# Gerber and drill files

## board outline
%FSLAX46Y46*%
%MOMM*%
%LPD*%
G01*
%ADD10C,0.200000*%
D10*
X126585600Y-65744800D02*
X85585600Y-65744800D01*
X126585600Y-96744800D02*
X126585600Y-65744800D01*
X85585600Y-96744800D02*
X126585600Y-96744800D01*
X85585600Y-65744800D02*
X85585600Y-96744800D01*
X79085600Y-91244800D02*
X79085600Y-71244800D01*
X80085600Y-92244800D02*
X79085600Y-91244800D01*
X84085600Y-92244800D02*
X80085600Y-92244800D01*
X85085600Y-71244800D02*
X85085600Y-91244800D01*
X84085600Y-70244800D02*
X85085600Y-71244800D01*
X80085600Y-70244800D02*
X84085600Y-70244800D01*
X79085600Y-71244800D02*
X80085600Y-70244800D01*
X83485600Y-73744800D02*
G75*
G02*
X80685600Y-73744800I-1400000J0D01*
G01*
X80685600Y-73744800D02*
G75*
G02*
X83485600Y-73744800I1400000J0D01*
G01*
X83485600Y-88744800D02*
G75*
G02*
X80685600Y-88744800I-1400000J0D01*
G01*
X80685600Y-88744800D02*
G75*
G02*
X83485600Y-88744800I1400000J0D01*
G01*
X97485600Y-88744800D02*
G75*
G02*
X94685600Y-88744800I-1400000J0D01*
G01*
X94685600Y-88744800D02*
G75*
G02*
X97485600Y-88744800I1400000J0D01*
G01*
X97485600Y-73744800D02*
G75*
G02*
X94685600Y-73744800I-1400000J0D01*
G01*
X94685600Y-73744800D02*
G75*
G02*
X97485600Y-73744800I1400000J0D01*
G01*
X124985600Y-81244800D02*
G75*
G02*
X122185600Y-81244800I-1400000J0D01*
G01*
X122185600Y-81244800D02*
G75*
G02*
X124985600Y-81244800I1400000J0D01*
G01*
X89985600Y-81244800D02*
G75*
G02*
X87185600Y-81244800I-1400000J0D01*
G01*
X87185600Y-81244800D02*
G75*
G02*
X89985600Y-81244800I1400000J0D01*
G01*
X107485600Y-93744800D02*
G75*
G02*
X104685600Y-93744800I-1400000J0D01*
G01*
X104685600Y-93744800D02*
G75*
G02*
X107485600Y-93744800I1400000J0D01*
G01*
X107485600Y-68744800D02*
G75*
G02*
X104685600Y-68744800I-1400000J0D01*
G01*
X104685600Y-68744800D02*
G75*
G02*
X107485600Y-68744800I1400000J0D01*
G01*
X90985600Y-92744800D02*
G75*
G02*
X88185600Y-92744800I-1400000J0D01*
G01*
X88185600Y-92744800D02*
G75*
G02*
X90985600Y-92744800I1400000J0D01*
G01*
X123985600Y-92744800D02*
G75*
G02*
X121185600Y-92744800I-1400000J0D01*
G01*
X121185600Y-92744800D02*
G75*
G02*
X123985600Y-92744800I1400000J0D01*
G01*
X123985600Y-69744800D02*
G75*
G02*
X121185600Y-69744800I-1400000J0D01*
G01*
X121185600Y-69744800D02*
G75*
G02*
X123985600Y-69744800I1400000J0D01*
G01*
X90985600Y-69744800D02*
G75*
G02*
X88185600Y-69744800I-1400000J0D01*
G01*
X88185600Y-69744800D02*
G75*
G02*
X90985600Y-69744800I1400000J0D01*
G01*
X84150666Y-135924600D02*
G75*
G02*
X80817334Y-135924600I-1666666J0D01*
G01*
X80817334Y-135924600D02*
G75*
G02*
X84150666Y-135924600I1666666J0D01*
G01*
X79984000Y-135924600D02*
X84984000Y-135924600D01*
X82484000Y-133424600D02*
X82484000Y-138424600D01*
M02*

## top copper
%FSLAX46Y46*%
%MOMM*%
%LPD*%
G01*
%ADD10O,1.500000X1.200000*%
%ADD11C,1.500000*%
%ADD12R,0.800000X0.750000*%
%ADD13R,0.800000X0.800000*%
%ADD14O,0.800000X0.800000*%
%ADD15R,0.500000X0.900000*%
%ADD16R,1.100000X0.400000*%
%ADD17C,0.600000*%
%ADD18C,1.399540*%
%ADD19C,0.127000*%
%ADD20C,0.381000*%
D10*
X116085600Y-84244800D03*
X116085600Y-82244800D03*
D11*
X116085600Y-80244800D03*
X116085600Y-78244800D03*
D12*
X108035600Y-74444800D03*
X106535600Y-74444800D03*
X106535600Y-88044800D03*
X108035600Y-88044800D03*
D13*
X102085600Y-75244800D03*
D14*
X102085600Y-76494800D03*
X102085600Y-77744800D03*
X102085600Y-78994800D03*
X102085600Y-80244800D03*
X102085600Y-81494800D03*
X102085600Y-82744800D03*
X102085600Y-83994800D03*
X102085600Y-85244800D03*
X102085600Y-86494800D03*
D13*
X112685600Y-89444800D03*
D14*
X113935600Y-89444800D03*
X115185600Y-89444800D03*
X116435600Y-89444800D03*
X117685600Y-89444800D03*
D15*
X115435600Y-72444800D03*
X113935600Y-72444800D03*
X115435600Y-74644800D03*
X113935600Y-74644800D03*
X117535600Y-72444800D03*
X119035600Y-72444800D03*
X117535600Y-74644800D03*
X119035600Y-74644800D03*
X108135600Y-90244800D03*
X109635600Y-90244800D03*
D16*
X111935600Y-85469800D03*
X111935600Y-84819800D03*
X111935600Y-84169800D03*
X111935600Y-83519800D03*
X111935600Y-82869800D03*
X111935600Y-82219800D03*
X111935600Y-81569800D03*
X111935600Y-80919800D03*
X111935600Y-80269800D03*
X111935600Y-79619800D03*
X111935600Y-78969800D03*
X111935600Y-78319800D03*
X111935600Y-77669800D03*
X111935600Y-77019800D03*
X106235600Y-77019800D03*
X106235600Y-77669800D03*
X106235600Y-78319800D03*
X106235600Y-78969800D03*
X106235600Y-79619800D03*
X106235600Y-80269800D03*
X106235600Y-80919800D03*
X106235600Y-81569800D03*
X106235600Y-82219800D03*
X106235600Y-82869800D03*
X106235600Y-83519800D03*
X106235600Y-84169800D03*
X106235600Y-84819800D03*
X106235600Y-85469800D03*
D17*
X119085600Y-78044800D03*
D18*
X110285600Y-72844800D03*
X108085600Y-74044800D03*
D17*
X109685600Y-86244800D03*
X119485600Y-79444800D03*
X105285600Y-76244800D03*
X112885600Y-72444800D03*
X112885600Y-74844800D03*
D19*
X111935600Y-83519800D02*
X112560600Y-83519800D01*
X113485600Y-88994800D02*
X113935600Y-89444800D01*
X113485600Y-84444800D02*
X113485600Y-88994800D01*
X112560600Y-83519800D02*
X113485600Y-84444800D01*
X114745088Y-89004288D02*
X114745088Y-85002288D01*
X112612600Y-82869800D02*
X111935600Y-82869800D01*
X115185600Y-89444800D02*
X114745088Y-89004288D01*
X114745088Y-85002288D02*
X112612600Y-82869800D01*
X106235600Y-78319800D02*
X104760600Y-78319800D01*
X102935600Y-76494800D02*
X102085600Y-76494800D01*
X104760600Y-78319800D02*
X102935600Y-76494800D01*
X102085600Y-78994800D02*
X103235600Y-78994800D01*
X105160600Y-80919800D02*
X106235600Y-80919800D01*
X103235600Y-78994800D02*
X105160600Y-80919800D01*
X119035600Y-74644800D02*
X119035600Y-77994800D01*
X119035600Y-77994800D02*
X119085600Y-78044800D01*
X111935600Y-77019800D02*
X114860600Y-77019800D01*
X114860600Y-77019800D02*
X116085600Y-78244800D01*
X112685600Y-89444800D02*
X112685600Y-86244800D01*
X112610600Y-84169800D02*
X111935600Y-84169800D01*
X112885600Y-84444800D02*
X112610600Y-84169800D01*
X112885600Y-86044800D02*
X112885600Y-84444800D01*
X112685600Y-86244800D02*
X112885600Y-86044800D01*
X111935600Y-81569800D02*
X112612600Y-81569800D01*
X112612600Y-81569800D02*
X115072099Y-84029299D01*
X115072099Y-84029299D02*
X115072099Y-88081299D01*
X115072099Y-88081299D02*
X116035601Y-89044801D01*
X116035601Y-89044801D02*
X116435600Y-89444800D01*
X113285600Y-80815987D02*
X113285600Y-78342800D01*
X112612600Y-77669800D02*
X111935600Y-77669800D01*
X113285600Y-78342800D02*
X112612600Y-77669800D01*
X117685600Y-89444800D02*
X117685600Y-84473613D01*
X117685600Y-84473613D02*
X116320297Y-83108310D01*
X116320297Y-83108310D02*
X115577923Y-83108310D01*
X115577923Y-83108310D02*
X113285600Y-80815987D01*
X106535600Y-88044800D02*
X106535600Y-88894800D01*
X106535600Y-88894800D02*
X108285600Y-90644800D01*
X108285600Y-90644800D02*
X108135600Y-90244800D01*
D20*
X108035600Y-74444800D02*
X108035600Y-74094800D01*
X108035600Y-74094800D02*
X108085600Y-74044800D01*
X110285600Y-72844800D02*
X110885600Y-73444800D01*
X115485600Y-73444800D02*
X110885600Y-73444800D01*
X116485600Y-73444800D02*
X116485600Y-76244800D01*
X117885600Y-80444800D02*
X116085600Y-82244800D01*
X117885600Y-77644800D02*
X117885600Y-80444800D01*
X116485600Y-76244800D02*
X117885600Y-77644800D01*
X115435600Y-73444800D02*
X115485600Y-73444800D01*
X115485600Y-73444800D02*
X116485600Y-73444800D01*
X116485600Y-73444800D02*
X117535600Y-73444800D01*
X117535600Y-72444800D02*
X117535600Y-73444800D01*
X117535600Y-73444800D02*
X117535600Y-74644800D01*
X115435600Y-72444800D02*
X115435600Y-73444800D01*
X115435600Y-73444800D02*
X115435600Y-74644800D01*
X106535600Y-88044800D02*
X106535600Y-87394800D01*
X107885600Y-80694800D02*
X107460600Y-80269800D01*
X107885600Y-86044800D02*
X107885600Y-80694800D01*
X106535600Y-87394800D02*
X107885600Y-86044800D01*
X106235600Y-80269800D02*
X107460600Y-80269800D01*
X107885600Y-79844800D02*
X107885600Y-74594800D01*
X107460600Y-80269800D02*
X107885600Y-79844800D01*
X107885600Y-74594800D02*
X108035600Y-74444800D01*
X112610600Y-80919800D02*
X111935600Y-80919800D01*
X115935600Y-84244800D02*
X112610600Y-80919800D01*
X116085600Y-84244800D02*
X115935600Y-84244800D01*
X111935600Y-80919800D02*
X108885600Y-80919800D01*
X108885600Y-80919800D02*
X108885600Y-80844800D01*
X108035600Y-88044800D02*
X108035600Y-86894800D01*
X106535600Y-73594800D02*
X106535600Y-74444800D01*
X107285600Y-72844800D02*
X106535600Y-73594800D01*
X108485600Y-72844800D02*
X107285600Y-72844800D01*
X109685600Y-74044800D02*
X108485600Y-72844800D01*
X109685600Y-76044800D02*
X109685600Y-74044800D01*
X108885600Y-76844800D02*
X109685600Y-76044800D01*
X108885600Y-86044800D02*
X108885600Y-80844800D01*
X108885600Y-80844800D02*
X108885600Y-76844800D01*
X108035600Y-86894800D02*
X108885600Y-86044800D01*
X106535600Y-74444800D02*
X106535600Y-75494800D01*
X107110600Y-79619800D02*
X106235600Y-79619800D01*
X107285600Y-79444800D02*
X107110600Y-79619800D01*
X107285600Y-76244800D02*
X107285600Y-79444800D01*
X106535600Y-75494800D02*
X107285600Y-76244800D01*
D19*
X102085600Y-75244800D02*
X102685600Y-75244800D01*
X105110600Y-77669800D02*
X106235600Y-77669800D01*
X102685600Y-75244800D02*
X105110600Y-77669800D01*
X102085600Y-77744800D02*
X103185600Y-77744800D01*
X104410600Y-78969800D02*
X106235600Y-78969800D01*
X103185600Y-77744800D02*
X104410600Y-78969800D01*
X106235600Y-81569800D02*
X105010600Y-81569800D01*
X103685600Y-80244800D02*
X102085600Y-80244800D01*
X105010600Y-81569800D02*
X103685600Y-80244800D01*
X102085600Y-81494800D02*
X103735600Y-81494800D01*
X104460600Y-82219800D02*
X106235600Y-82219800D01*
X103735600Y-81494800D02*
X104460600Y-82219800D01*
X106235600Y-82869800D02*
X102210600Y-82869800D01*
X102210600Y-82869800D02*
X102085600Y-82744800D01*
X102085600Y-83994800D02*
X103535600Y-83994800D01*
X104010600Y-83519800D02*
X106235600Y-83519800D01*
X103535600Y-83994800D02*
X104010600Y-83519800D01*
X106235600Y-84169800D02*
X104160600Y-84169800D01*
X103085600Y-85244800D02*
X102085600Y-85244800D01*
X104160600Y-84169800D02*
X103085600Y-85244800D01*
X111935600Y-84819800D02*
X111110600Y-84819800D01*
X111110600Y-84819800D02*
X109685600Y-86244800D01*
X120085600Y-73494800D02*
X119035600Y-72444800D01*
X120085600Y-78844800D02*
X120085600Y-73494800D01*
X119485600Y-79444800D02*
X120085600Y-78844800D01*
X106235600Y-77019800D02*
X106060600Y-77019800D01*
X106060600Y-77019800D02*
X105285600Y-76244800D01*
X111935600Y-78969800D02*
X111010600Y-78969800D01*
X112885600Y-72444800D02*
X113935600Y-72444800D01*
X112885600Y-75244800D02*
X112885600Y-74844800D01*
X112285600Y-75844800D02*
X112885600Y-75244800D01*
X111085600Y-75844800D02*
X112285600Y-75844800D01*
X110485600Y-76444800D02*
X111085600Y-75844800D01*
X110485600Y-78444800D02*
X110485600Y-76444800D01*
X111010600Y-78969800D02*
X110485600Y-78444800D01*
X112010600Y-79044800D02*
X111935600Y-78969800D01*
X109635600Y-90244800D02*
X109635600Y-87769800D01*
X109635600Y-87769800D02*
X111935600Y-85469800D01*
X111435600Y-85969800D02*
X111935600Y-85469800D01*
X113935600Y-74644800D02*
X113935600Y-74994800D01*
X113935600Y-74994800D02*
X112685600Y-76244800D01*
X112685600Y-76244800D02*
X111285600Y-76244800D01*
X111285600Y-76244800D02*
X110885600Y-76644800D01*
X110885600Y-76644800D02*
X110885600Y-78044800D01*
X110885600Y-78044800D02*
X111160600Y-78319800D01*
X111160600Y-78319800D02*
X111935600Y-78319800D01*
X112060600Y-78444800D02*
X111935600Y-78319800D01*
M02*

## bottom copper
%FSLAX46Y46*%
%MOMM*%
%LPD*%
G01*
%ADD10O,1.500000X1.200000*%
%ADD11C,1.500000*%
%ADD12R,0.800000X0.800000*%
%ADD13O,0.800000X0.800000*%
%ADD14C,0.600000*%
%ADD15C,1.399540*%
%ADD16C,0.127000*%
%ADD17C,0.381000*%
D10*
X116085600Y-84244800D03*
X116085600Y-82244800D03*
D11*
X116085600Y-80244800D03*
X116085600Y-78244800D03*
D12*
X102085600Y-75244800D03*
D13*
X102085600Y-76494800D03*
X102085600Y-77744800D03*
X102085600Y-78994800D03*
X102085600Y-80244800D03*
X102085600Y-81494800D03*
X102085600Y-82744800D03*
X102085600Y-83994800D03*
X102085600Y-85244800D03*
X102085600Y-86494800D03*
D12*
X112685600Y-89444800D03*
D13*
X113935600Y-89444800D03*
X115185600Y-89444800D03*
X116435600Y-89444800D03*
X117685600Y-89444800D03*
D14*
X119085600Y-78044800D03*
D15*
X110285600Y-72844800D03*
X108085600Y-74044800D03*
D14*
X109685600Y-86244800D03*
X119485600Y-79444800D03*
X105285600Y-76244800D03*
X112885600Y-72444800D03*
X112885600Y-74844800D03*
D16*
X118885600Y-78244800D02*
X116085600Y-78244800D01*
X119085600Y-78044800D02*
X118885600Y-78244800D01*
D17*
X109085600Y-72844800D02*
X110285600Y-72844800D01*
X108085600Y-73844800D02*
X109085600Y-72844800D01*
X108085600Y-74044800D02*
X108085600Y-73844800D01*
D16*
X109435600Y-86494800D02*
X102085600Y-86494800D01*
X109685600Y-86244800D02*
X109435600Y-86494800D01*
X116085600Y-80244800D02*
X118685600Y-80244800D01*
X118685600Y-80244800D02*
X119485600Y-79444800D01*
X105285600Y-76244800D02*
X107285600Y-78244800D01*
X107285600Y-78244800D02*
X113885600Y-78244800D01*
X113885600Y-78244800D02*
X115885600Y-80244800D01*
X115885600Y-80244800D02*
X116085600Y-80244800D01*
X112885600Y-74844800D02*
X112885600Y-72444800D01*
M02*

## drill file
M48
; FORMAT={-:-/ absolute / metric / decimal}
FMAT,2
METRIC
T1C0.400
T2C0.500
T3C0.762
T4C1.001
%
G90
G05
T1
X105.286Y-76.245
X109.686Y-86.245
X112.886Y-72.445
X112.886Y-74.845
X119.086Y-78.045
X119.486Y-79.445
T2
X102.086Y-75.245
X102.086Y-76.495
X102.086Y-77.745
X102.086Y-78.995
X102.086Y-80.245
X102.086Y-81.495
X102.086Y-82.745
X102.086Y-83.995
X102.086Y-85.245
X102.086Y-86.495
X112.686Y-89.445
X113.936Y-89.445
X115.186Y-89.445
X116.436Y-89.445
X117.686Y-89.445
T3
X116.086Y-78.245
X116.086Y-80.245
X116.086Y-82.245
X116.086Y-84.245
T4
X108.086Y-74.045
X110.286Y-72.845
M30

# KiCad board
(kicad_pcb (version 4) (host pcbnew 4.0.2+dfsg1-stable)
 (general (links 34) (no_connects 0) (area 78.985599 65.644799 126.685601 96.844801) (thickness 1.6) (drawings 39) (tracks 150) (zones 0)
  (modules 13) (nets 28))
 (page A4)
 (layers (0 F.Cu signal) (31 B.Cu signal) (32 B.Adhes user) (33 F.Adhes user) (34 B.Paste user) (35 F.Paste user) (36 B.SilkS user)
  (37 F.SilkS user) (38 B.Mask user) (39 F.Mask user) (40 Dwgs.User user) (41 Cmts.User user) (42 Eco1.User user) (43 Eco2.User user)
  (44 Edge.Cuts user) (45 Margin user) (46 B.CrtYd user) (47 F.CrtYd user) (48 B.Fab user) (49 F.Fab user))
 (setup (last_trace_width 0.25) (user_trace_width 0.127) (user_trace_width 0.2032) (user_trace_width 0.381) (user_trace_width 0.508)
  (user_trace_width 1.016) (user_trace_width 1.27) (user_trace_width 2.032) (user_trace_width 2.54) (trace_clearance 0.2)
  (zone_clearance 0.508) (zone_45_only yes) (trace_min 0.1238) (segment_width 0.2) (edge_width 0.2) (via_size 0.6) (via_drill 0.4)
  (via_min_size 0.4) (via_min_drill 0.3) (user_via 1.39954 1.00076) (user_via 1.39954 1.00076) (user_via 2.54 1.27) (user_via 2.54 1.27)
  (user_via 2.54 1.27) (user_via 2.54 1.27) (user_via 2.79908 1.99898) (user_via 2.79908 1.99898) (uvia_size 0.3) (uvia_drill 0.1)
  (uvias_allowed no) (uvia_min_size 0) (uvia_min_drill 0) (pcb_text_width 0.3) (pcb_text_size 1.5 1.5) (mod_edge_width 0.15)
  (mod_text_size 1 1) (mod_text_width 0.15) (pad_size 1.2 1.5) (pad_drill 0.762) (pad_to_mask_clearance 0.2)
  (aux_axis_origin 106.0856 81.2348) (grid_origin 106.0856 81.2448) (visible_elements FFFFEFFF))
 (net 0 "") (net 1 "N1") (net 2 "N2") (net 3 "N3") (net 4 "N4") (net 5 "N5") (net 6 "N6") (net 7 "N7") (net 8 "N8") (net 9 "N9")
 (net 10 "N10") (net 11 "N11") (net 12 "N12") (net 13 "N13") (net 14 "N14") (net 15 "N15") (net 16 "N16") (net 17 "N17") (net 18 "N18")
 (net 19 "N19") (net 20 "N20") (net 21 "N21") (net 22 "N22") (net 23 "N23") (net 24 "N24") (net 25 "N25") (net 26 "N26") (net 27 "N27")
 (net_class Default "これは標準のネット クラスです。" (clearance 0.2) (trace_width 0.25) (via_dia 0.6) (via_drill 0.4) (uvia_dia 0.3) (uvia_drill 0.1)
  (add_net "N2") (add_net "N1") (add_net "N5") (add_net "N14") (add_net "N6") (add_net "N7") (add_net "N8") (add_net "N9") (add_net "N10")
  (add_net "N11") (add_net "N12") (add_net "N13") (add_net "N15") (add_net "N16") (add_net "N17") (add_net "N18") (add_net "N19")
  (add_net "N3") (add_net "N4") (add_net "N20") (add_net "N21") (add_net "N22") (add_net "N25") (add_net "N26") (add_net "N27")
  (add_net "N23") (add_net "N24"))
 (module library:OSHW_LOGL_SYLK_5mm (layer F.Cu) (at 82.0856 81.2448 270)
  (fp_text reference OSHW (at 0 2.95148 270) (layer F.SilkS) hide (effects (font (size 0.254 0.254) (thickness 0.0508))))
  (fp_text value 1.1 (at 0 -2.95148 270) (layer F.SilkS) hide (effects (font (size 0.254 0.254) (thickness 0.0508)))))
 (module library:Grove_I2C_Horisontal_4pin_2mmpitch (layer F.Cu) (at 116.0856 81.2448 90)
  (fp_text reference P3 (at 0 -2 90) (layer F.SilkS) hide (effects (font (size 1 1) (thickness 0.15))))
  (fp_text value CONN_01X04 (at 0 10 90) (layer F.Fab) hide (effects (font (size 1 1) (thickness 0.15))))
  (pad 1 thru_hole oval (at -3 0 90) (size 1.2 1.5) (drill 0.762) (layers *.Cu *.Mask F.SilkS) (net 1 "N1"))
  (pad 2 thru_hole oval (at -1 0 90) (size 1.2 1.5) (drill 0.762) (layers *.Cu *.Mask F.SilkS) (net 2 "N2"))
  (pad 3 thru_hole circle (at 1 0 90) (size 1.5 1.5) (drill 0.762) (layers *.Cu *.Mask F.SilkS) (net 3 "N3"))
  (pad 4 thru_hole circle (at 3 0 90) (size 1.5 1.5) (drill 0.762) (layers *.Cu *.Mask F.SilkS) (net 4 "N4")))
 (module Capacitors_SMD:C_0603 (layer F.Cu) (at 107.2856 74.4448 180)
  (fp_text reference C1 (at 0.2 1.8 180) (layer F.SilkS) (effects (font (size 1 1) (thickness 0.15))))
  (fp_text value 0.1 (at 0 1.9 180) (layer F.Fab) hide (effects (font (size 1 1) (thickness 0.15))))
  (pad 1 smd rect (at -0.75 0 180) (size 0.8 0.75) (layers F.Cu F.Paste F.Mask) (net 2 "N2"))
  (pad 2 smd rect (at 0.75 0 180) (size 0.8 0.75) (layers F.Cu F.Paste F.Mask) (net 1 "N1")))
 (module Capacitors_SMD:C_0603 (layer F.Cu) (at 107.2856 88.0448)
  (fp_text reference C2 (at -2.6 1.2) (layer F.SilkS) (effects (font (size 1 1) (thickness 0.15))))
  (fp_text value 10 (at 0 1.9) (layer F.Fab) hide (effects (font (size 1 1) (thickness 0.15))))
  (pad 1 smd rect (at -0.75 0) (size 0.8 0.75) (layers F.Cu F.Paste F.Mask) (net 2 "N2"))
  (pad 2 smd rect (at 0.75 0) (size 0.8 0.75) (layers F.Cu F.Paste F.Mask) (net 1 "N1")))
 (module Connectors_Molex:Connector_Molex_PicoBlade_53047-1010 (layer F.Cu) (at 102.0856 75.2448 270)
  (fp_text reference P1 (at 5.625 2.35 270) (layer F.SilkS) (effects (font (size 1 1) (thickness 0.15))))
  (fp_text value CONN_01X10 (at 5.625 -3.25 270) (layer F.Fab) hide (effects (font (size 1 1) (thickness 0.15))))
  (pad 1 thru_hole rect (at 0 0 270) (size 0.8 0.8) (drill 0.5) (layers *.Cu *.Mask F.SilkS) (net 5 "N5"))
  (pad 2 thru_hole oval (at 1.25 0 270) (size 0.8 0.8) (drill 0.5) (layers *.Cu *.Mask F.SilkS) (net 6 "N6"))
  (pad 3 thru_hole oval (at 2.5 0 270) (size 0.8 0.8) (drill 0.5) (layers *.Cu *.Mask F.SilkS) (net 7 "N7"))
  (pad 4 thru_hole oval (at 3.75 0 270) (size 0.8 0.8) (drill 0.5) (layers *.Cu *.Mask F.SilkS) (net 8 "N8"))
  (pad 5 thru_hole oval (at 5 0 270) (size 0.8 0.8) (drill 0.5) (layers *.Cu *.Mask F.SilkS) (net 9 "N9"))
  (pad 6 thru_hole oval (at 6.25 0 270) (size 0.8 0.8) (drill 0.5) (layers *.Cu *.Mask F.SilkS) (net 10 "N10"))
  (pad 7 thru_hole oval (at 7.5 0 270) (size 0.8 0.8) (drill 0.5) (layers *.Cu *.Mask F.SilkS) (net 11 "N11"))
  (pad 8 thru_hole oval (at 8.75 0 270) (size 0.8 0.8) (drill 0.5) (layers *.Cu *.Mask F.SilkS) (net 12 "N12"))
  (pad 9 thru_hole oval (at 10 0 270) (size 0.8 0.8) (drill 0.5) (layers *.Cu *.Mask F.SilkS) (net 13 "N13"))
  (pad 10 thru_hole oval (at 11.25 0 270) (size 0.8 0.8) (drill 0.5) (layers *.Cu *.Mask F.SilkS) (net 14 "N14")))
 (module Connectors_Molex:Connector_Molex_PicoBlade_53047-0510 (layer F.Cu) (at 112.6856 89.4448)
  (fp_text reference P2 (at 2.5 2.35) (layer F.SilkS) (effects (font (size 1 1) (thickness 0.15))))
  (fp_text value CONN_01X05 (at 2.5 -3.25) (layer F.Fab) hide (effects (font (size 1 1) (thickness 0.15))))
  (pad 1 thru_hole rect (at 0 0) (size 0.8 0.8) (drill 0.5) (layers *.Cu *.Mask F.SilkS) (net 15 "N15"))
  (pad 2 thru_hole oval (at 1.25 0) (size 0.8 0.8) (drill 0.5) (layers *.Cu *.Mask F.SilkS) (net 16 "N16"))
  (pad 3 thru_hole oval (at 2.5 0) (size 0.8 0.8) (drill 0.5) (layers *.Cu *.Mask F.SilkS) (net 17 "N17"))
  (pad 4 thru_hole oval (at 3.75 0) (size 0.8 0.8) (drill 0.5) (layers *.Cu *.Mask F.SilkS) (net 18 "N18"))
  (pad 5 thru_hole oval (at 5 0) (size 0.8 0.8) (drill 0.5) (layers *.Cu *.Mask F.SilkS) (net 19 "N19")))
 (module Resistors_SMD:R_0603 (layer F.Cu) (at 114.6856 72.4448 180)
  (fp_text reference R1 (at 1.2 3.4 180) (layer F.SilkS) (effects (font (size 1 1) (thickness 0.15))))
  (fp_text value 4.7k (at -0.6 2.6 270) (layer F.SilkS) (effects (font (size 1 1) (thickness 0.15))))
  (pad 1 smd rect (at -0.75 0 180) (size 0.5 0.9) (layers F.Cu F.Paste F.Mask) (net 2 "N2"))
  (pad 2 smd rect (at 0.75 0 180) (size 0.5 0.9) (layers F.Cu F.Paste F.Mask) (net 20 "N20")))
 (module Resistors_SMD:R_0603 (layer F.Cu) (at 114.6856 74.6448 180)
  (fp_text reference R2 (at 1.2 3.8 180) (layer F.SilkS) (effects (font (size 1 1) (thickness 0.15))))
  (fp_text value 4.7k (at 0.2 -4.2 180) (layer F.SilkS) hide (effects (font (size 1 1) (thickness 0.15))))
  (pad 1 smd rect (at -0.75 0 180) (size 0.5 0.9) (layers F.Cu F.Paste F.Mask) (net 2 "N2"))
  (pad 2 smd rect (at 0.75 0 180) (size 0.5 0.9) (layers F.Cu F.Paste F.Mask) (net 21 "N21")))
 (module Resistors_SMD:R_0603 (layer F.Cu) (at 118.2856 72.4448)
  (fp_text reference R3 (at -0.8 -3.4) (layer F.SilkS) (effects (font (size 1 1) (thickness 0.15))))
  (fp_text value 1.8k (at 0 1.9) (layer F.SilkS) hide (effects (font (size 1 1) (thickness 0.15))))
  (pad 1 smd rect (at -0.75 0) (size 0.5 0.9) (layers F.Cu F.Paste F.Mask) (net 2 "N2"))
  (pad 2 smd rect (at 0.75 0) (size 0.5 0.9) (layers F.Cu F.Paste F.Mask) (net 3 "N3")))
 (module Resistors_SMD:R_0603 (layer F.Cu) (at 118.2856 74.6448)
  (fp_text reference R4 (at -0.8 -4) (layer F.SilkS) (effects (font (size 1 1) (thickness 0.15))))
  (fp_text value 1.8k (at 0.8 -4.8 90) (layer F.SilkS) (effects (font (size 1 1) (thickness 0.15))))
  (pad 1 smd rect (at -0.75 0) (size 0.5 0.9) (layers F.Cu F.Paste F.Mask) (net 2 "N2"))
  (pad 2 smd rect (at 0.75 0) (size 0.5 0.9) (layers F.Cu F.Paste F.Mask) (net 4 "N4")))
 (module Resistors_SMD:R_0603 (layer F.Cu) (at 108.8856 90.2448)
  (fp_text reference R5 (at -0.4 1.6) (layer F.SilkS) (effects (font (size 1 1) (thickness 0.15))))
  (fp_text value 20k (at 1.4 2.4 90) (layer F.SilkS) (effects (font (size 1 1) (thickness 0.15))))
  (pad 1 smd rect (at -0.75 0) (size 0.5 0.9) (layers F.Cu F.Paste F.Mask) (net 2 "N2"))
  (pad 2 smd rect (at 0.75 0) (size 0.5 0.9) (layers F.Cu F.Paste F.Mask) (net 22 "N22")))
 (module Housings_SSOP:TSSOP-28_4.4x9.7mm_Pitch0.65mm (layer F.Cu) (at 109.0856 81.2448 180)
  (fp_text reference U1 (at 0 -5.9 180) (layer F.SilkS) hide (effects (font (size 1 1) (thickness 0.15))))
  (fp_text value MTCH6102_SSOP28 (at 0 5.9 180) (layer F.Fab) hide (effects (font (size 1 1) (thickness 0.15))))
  (pad 1 smd rect (at -2.85 -4.225 180) (size 1.1 0.4) (layers F.Cu F.Paste F.Mask) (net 22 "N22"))
  (pad 2 smd rect (at -2.85 -3.575 180) (size 1.1 0.4) (layers F.Cu F.Paste F.Mask) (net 14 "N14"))
  (pad 3 smd rect (at -2.85 -2.925 180) (size 1.1 0.4) (layers F.Cu F.Paste F.Mask) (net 15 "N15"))
  (pad 4 smd rect (at -2.85 -2.275 180) (size 1.1 0.4) (layers F.Cu F.Paste F.Mask) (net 16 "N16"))
  (pad 5 smd rect (at -2.85 -1.625 180) (size 1.1 0.4) (layers F.Cu F.Paste F.Mask) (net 17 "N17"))
  (pad 6 smd rect (at -2.85 -0.975 180) (size 1.1 0.4) (layers F.Cu F.Paste F.Mask) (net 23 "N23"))
  (pad 7 smd rect (at -2.85 -0.325 180) (size 1.1 0.4) (layers F.Cu F.Paste F.Mask) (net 18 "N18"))
  (pad 8 smd rect (at -2.85 0.325 180) (size 1.1 0.4) (layers F.Cu F.Paste F.Mask) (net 1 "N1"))
  (pad 9 smd rect (at -2.85 0.975 180) (size 1.1 0.4) (layers F.Cu F.Paste F.Mask) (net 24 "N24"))
  (pad 10 smd rect (at -2.85 1.625 180) (size 1.1 0.4) (layers F.Cu F.Paste F.Mask) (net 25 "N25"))
  (pad 11 smd rect (at -2.85 2.275 180) (size 1.1 0.4) (layers F.Cu F.Paste F.Mask) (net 20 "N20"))
  (pad 12 smd rect (at -2.85 2.925 180) (size 1.1 0.4) (layers F.Cu F.Paste F.Mask) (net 21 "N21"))
  (pad 13 smd rect (at -2.85 3.575 180) (size 1.1 0.4) (layers F.Cu F.Paste F.Mask) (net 19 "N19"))
  (pad 14 smd rect (at -2.85 4.225 180) (size 1.1 0.4) (layers F.Cu F.Paste F.Mask) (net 4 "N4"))
  (pad 15 smd rect (at 2.85 4.225 180) (size 1.1 0.4) (layers F.Cu F.Paste F.Mask) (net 3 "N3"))
  (pad 16 smd rect (at 2.85 3.575 180) (size 1.1 0.4) (layers F.Cu F.Paste F.Mask) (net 5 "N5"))
  (pad 17 smd rect (at 2.85 2.925 180) (size 1.1 0.4) (layers F.Cu F.Paste F.Mask) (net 6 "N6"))
  (pad 18 smd rect (at 2.85 2.275 180) (size 1.1 0.4) (layers F.Cu F.Paste F.Mask) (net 7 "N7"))
  (pad 19 smd rect (at 2.85 1.625 180) (size 1.1 0.4) (layers F.Cu F.Paste F.Mask) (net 1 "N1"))
  (pad 20 smd rect (at 2.85 0.975 180) (size 1.1 0.4) (layers F.Cu F.Paste F.Mask) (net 2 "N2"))
  (pad 21 smd rect (at 2.85 0.325 180) (size 1.1 0.4) (layers F.Cu F.Paste F.Mask) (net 8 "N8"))
  (pad 22 smd rect (at 2.85 -0.325 180) (size 1.1 0.4) (layers F.Cu F.Paste F.Mask) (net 9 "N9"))
  (pad 23 smd rect (at 2.85 -0.975 180) (size 1.1 0.4) (layers F.Cu F.Paste F.Mask) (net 10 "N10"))
  (pad 24 smd rect (at 2.85 -1.625 180) (size 1.1 0.4) (layers F.Cu F.Paste F.Mask) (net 11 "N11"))
  (pad 25 smd rect (at 2.85 -2.275 180) (size 1.1 0.4) (layers F.Cu F.Paste F.Mask) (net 12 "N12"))
  (pad 26 smd rect (at 2.85 -2.925 180) (size 1.1 0.4) (layers F.Cu F.Paste F.Mask) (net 13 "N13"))
  (pad 27 smd rect (at 2.85 -3.575 180) (size 1.1 0.4) (layers F.Cu F.Paste F.Mask) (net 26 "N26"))
  (pad 28 smd rect (at 2.85 -4.225 180) (size 1.1 0.4) (layers F.Cu F.Paste F.Mask) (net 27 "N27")))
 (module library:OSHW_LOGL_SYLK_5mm (layer F.Cu) (at 96.0856 81.2448 270)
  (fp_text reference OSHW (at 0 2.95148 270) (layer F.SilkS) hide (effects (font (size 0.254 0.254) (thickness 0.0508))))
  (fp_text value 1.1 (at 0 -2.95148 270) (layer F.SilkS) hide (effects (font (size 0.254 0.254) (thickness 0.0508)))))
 (gr_line (start 126.5856 65.7448) (end 85.5856 65.7448) (angle 90) (layer Edge.Cuts) (width 0.2))
 (gr_line (start 126.5856 96.7448) (end 126.5856 65.7448) (angle 90) (layer Edge.Cuts) (width 0.2))
 (gr_line (start 85.5856 96.7448) (end 126.5856 96.7448) (angle 90) (layer Edge.Cuts) (width 0.2))
 (gr_line (start 85.5856 65.7448) (end 85.5856 96.7448) (angle 90) (layer Edge.Cuts) (width 0.2))
 (gr_line (start 79.0856 91.2448) (end 79.0856 71.2448) (angle 90) (layer Edge.Cuts) (width 0.2))
 (gr_line (start 80.0856 92.2448) (end 79.0856 91.2448) (angle 90) (layer Edge.Cuts) (width 0.2))
 (gr_line (start 84.0856 92.2448) (end 80.0856 92.2448) (angle 90) (layer Edge.Cuts) (width 0.2))
 (gr_line (start 85.0856 71.2448) (end 85.0856 91.2448) (angle 90) (layer Edge.Cuts) (width 0.2))
 (gr_line (start 84.0856 70.2448) (end 85.0856 71.2448) (angle 90) (layer Edge.Cuts) (width 0.2))
 (gr_line (start 80.0856 70.2448) (end 84.0856 70.2448) (angle 90) (layer Edge.Cuts) (width 0.2))
 (gr_line (start 79.0856 71.2448) (end 80.0856 70.2448) (angle 90) (layer Edge.Cuts) (width 0.2))
 (gr_circle (center 82.0856 73.7448) (end 83.4856 73.7448) (layer Edge.Cuts) (width 0.2))
 (gr_circle (center 82.0856 88.7448) (end 83.4856 88.7448) (layer Edge.Cuts) (width 0.2))
 (gr_circle (center 96.0856 88.7448) (end 97.4856 88.7448) (layer Edge.Cuts) (width 0.2))
 (gr_circle (center 96.0856 73.7448) (end 97.4856 73.7448) (layer Edge.Cuts) (width 0.2))
 (gr_circle (center 123.5856 81.2448) (end 124.9856 81.2448) (layer Edge.Cuts) (width 0.2))
 (gr_circle (center 88.5856 81.2448) (end 89.9856 81.2448) (layer Edge.Cuts) (width 0.2))
 (gr_circle (center 106.0856 93.7448) (end 107.4856 93.7448) (layer Edge.Cuts) (width 0.2))
 (gr_circle (center 106.0856 68.7448) (end 107.4856 68.7448) (layer Edge.Cuts) (width 0.2))
 (gr_circle (center 89.5856 92.7448) (end 90.9856 92.7448) (layer Edge.Cuts) (width 0.2))
 (gr_circle (center 122.5856 92.7448) (end 123.9856 92.7448) (layer Edge.Cuts) (width 0.2))
 (gr_circle (center 122.5856 69.7448) (end 123.9856 69.7448) (layer Edge.Cuts) (width 0.2))
 (gr_circle (center 89.5856 69.7448) (end 90.9856 69.7448) (layer Edge.Cuts) (width 0.2))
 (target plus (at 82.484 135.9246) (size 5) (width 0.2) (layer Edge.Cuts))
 (segment (start 111.9356 83.5198) (end 112.5606 83.5198) (width 0.127) (layer F.Cu) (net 16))
 (segment (start 113.4856 88.9948) (end 113.9356 89.4448) (width 0.127) (layer F.Cu) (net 16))
 (segment (start 113.4856 84.4448) (end 113.4856 88.9948) (width 0.127) (layer F.Cu) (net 16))
 (segment (start 112.5606 83.5198) (end 113.4856 84.4448) (width 0.127) (layer F.Cu) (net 16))
 (segment (start 114.745088 89.004288) (end 114.745088 85.002288) (width 0.127) (layer F.Cu) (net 17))
 (segment (start 112.6126 82.8698) (end 111.9356 82.8698) (width 0.127) (layer F.Cu) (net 17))
 (segment (start 115.1856 89.4448) (end 114.745088 89.004288) (width 0.127) (layer F.Cu) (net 17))
 (segment (start 114.745088 85.002288) (end 112.6126 82.8698) (width 0.127) (layer F.Cu) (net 17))
 (segment (start 106.2356 78.3198) (end 104.7606 78.3198) (width 0.127) (layer F.Cu) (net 6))
 (segment (start 102.9356 76.4948) (end 102.0856 76.4948) (width 0.127) (layer F.Cu) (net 6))
 (segment (start 104.7606 78.3198) (end 102.9356 76.4948) (width 0.127) (layer F.Cu) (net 6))
 (segment (start 102.0856 78.9948) (end 103.2356 78.9948) (width 0.127) (layer F.Cu) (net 8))
 (segment (start 105.1606 80.9198) (end 106.2356 80.9198) (width 0.127) (layer F.Cu) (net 8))
 (segment (start 103.2356 78.9948) (end 105.1606 80.9198) (width 0.127) (layer F.Cu) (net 8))
 (segment (start 119.0356 74.6448) (end 119.0356 77.9948) (width 0.127) (layer F.Cu) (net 4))
 (segment (start 118.8856 78.2448) (end 116.0856 78.2448) (width 0.127) (layer B.Cu) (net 4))
 (segment (start 119.0856 78.0448) (end 118.8856 78.2448) (width 0.127) (layer B.Cu) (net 4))
 (via (at 119.0856 78.0448) (size 0.6) (drill 0.4) (layers F.Cu B.Cu) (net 4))
 (segment (start 119.0356 77.9948) (end 119.0856 78.0448) (width 0.127) (layer F.Cu) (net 4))
 (segment (start 111.9356 77.0198) (end 114.8606 77.0198) (width 0.127) (layer F.Cu) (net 4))
 (segment (start 114.8606 77.0198) (end 116.0856 78.2448) (width 0.127) (layer F.Cu) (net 4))
 (segment (start 112.6856 89.4448) (end 112.6856 86.2448) (width 0.127) (layer F.Cu) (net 15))
 (segment (start 112.6106 84.1698) (end 111.9356 84.1698) (width 0.127) (layer F.Cu) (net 15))
 (segment (start 112.8856 84.4448) (end 112.6106 84.1698) (width 0.127) (layer F.Cu) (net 15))
 (segment (start 112.8856 86.0448) (end 112.8856 84.4448) (width 0.127) (layer F.Cu) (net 15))
 (segment (start 112.6856 86.2448) (end 112.8856 86.0448) (width 0.127) (layer F.Cu) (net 15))
 (segment (start 111.9356 81.5698) (end 112.6126 81.5698) (width 0.127) (layer F.Cu) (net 18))
 (segment (start 112.6126 81.5698) (end 115.072099 84.029299) (width 0.127) (layer F.Cu) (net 18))
 (segment (start 115.072099 84.029299) (end 115.072099 88.081299) (width 0.127) (layer F.Cu) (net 18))
 (segment (start 115.072099 88.081299) (end 116.035601 89.044801) (width 0.127) (layer F.Cu) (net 18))
 (segment (start 116.035601 89.044801) (end 116.4356 89.4448) (width 0.127) (layer F.Cu) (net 18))
 (segment (start 113.2856 80.815987) (end 113.2856 78.3428) (width 0.127) (layer F.Cu) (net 19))
 (segment (start 112.6126 77.6698) (end 111.9356 77.6698) (width 0.127) (layer F.Cu) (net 19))
 (segment (start 113.2856 78.3428) (end 112.6126 77.6698) (width 0.127) (layer F.Cu) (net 19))
 (segment (start 117.6856 89.4448) (end 117.6856 84.473613) (width 0.127) (layer F.Cu) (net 19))
 (segment (start 117.6856 84.473613) (end 116.320297 83.10831) (width 0.127) (layer F.Cu) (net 19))
 (segment (start 116.320297 83.10831) (end 115.577923 83.10831) (width 0.127) (layer F.Cu) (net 19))
 (segment (start 115.577923 83.10831) (end 113.2856 80.815987) (width 0.127) (layer F.Cu) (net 19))
 (segment (start 106.5356 88.0448) (end 106.5356 88.8948) (width 0.127) (layer F.Cu) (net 2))
 (segment (start 106.5356 88.8948) (end 108.2856 90.6448) (width 0.127) (layer F.Cu) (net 2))
 (segment (start 108.2856 90.6448) (end 108.1356 90.2448) (width 0.127) (layer F.Cu) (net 2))
 (segment (start 108.0356 74.4448) (end 108.0356 74.0948) (width 0.381) (layer F.Cu) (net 2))
 (segment (start 108.0356 74.0948) (end 108.0856 74.0448) (width 0.381) (layer F.Cu) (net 2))
 (segment (start 110.2856 72.8448) (end 110.8856 73.4448) (width 0.381) (layer F.Cu) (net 2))
 (via (at 110.2856 72.8448) (size 1.39954) (drill 1.00076) (layers F.Cu B.Cu) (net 2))
 (segment (start 109.0856 72.8448) (end 110.2856 72.8448) (width 0.381) (layer B.Cu) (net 2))
 (segment (start 108.0856 73.8448) (end 109.0856 72.8448) (width 0.381) (layer B.Cu) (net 2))
 (segment (start 108.0856 74.0448) (end 108.0856 73.8448) (width 0.381) (layer B.Cu) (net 2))
 (via (at 108.0856 74.0448) (size 1.39954) (drill 1.00076) (layers F.Cu B.Cu) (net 2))
 (segment (start 115.4856 73.4448) (end 110.8856 73.4448) (width 0.381) (layer F.Cu) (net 2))
 (segment (start 116.4856 73.4448) (end 116.4856 76.2448) (width 0.381) (layer F.Cu) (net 2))
 (segment (start 117.8856 80.4448) (end 116.0856 82.2448) (width 0.381) (layer F.Cu) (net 2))
 (segment (start 117.8856 77.6448) (end 117.8856 80.4448) (width 0.381) (layer F.Cu) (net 2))
 (segment (start 116.4856 76.2448) (end 117.8856 77.6448) (width 0.381) (layer F.Cu) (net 2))
 (segment (start 115.4356 73.4448) (end 115.4856 73.4448) (width 0.381) (layer F.Cu) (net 2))
 (segment (start 115.4856 73.4448) (end 116.4856 73.4448) (width 0.381) (layer F.Cu) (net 2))
 (segment (start 116.4856 73.4448) (end 117.5356 73.4448) (width 0.381) (layer F.Cu) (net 2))
 (segment (start 117.5356 72.4448) (end 117.5356 73.4448) (width 0.381) (layer F.Cu) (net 2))
 (segment (start 117.5356 73.4448) (end 117.5356 74.6448) (width 0.381) (layer F.Cu) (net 2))
 (segment (start 115.4356 72.4448) (end 115.4356 73.4448) (width 0.381) (layer F.Cu) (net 2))
 (segment (start 115.4356 73.4448) (end 115.4356 74.6448) (width 0.381) (layer F.Cu) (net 2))
 (segment (start 106.5356 88.0448) (end 106.5356 87.3948) (width 0.381) (layer F.Cu) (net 2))
 (segment (start 107.8856 80.6948) (end 107.4606 80.2698) (width 0.381) (layer F.Cu) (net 2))
 (segment (start 107.8856 86.0448) (end 107.8856 80.6948) (width 0.381) (layer F.Cu) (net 2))
 (segment (start 106.5356 87.3948) (end 107.8856 86.0448) (width 0.381) (layer F.Cu) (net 2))
 (segment (start 106.2356 80.2698) (end 107.4606 80.2698) (width 0.381) (layer F.Cu) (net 2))
 (segment (start 107.8856 79.8448) (end 107.8856 74.5948) (width 0.381) (layer F.Cu) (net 2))
 (segment (start 107.4606 80.2698) (end 107.8856 79.8448) (width 0.381) (layer F.Cu) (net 2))
 (segment (start 107.8856 74.5948) (end 108.0356 74.4448) (width 0.381) (layer F.Cu) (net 2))
 (segment (start 112.6106 80.9198) (end 111.9356 80.9198) (width 0.381) (layer F.Cu) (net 1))
 (segment (start 115.9356 84.2448) (end 112.6106 80.9198) (width 0.381) (layer F.Cu) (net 1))
 (segment (start 116.0856 84.2448) (end 115.9356 84.2448) (width 0.381) (layer F.Cu) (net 1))
 (segment (start 111.9356 80.9198) (end 108.8856 80.9198) (width 0.381) (layer F.Cu) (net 1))
 (segment (start 108.8856 80.9198) (end 108.8856 80.8448) (width 0.381) (layer F.Cu) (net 1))
 (segment (start 108.0356 88.0448) (end 108.0356 86.8948) (width 0.381) (layer F.Cu) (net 1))
 (segment (start 106.5356 73.5948) (end 106.5356 74.4448) (width 0.381) (layer F.Cu) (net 1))
 (segment (start 107.2856 72.8448) (end 106.5356 73.5948) (width 0.381) (layer F.Cu) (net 1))
 (segment (start 108.4856 72.8448) (end 107.2856 72.8448) (width 0.381) (layer F.Cu) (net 1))
 (segment (start 109.6856 74.0448) (end 108.4856 72.8448) (width 0.381) (layer F.Cu) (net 1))
 (segment (start 109.6856 76.0448) (end 109.6856 74.0448) (width 0.381) (layer F.Cu) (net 1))
 (segment (start 108.8856 76.8448) (end 109.6856 76.0448) (width 0.381) (layer F.Cu) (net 1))
 (segment (start 108.8856 86.0448) (end 108.8856 80.8448) (width 0.381) (layer F.Cu) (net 1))
 (segment (start 108.8856 80.8448) (end 108.8856 76.8448) (width 0.381) (layer F.Cu) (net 1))
 (segment (start 108.0356 86.8948) (end 108.8856 86.0448) (width 0.381) (layer F.Cu) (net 1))
 (segment (start 106.5356 74.4448) (end 106.5356 75.4948) (width 0.381) (layer F.Cu) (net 1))
 (segment (start 107.1106 79.6198) (end 106.2356 79.6198) (width 0.381) (layer F.Cu) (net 1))
 (segment (start 107.2856 79.4448) (end 107.1106 79.6198) (width 0.381) (layer F.Cu) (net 1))
 (segment (start 107.2856 76.2448) (end 107.2856 79.4448) (width 0.381) (layer F.Cu) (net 1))
 (segment (start 106.5356 75.4948) (end 107.2856 76.2448) (width 0.381) (layer F.Cu) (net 1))
 (segment (start 102.0856 75.2448) (end 102.6856 75.2448) (width 0.127) (layer F.Cu) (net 5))
 (segment (start 105.1106 77.6698) (end 106.2356 77.6698) (width 0.127) (layer F.Cu) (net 5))
 (segment (start 102.6856 75.2448) (end 105.1106 77.6698) (width 0.127) (layer F.Cu) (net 5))
 (segment (start 102.0856 77.7448) (end 103.1856 77.7448) (width 0.127) (layer F.Cu) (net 7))
 (segment (start 104.4106 78.9698) (end 106.2356 78.9698) (width 0.127) (layer F.Cu) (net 7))
 (segment (start 103.1856 77.7448) (end 104.4106 78.9698) (width 0.127) (layer F.Cu) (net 7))
 (segment (start 106.2356 81.5698) (end 105.0106 81.5698) (width 0.127) (layer F.Cu) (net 9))
 (segment (start 103.6856 80.2448) (end 102.0856 80.2448) (width 0.127) (layer F.Cu) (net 9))
 (segment (start 105.0106 81.5698) (end 103.6856 80.2448) (width 0.127) (layer F.Cu) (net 9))
 (segment (start 102.0856 81.4948) (end 103.7356 81.4948) (width 0.127) (layer F.Cu) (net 10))
 (segment (start 104.4606 82.2198) (end 106.2356 82.2198) (width 0.127) (layer F.Cu) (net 10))
 (segment (start 103.7356 81.4948) (end 104.4606 82.2198) (width 0.127) (layer F.Cu) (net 10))
 (segment (start 106.2356 82.8698) (end 102.2106 82.8698) (width 0.127) (layer F.Cu) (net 11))
 (segment (start 102.2106 82.8698) (end 102.0856 82.7448) (width 0.127) (layer F.Cu) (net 11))
 (segment (start 102.0856 83.9948) (end 103.5356 83.9948) (width 0.127) (layer F.Cu) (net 12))
 (segment (start 104.0106 83.5198) (end 106.2356 83.5198) (width 0.127) (layer F.Cu) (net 12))
 (segment (start 103.5356 83.9948) (end 104.0106 83.5198) (width 0.127) (layer F.Cu) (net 12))
 (segment (start 106.2356 84.1698) (end 104.1606 84.1698) (width 0.127) (layer F.Cu) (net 13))
 (segment (start 103.0856 85.2448) (end 102.0856 85.2448) (width 0.127) (layer F.Cu) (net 13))
 (segment (start 104.1606 84.1698) (end 103.0856 85.2448) (width 0.127) (layer F.Cu) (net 13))
 (segment (start 111.9356 84.8198) (end 111.1106 84.8198) (width 0.127) (layer F.Cu) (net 14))
 (segment (start 109.4356 86.4948) (end 102.0856 86.4948) (width 0.127) (layer B.Cu) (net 14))
 (segment (start 109.6856 86.2448) (end 109.4356 86.4948) (width 0.127) (layer B.Cu) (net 14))
 (via (at 109.6856 86.2448) (size 0.6) (drill 0.4) (layers F.Cu B.Cu) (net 14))
 (segment (start 111.1106 84.8198) (end 109.6856 86.2448) (width 0.127) (layer F.Cu) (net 14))
 (segment (start 116.0856 80.2448) (end 118.6856 80.2448) (width 0.127) (layer B.Cu) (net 3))
 (segment (start 120.0856 73.4948) (end 119.0356 72.4448) (width 0.127) (layer F.Cu) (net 3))
 (segment (start 120.0856 78.8448) (end 120.0856 73.4948) (width 0.127) (layer F.Cu) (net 3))
 (segment (start 119.4856 79.4448) (end 120.0856 78.8448) (width 0.127) (layer F.Cu) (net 3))
 (via (at 119.4856 79.4448) (size 0.6) (drill 0.4) (layers F.Cu B.Cu) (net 3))
 (segment (start 118.6856 80.2448) (end 119.4856 79.4448) (width 0.127) (layer B.Cu) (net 3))
 (segment (start 106.2356 77.0198) (end 106.0606 77.0198) (width 0.127) (layer F.Cu) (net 3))
 (segment (start 106.0606 77.0198) (end 105.2856 76.2448) (width 0.127) (layer F.Cu) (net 3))
 (via (at 105.2856 76.2448) (size 0.6) (drill 0.4) (layers F.Cu B.Cu) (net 3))
 (segment (start 105.2856 76.2448) (end 107.2856 78.2448) (width 0.127) (layer B.Cu) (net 3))
 (segment (start 107.2856 78.2448) (end 113.8856 78.2448) (width 0.127) (layer B.Cu) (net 3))
 (segment (start 113.8856 78.2448) (end 115.8856 80.2448) (width 0.127) (layer B.Cu) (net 3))
 (segment (start 115.8856 80.2448) (end 116.0856 80.2448) (width 0.127) (layer B.Cu) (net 3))
 (segment (start 111.9356 78.9698) (end 111.0106 78.9698) (width 0.127) (layer F.Cu) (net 20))
 (segment (start 112.8856 72.4448) (end 113.9356 72.4448) (width 0.127) (layer F.Cu) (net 20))
 (via (at 112.8856 72.4448) (size 0.6) (drill 0.4) (layers F.Cu B.Cu) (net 20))
 (segment (start 112.8856 74.8448) (end 112.8856 72.4448) (width 0.127) (layer B.Cu) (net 20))
 (via (at 112.8856 74.8448) (size 0.6) (drill 0.4) (layers F.Cu B.Cu) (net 20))
 (segment (start 112.8856 75.2448) (end 112.8856 74.8448) (width 0.127) (layer F.Cu) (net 20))
 (segment (start 112.2856 75.8448) (end 112.8856 75.2448) (width 0.127) (layer F.Cu) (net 20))
 (segment (start 111.0856 75.8448) (end 112.2856 75.8448) (width 0.127) (layer F.Cu) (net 20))
 (segment (start 110.4856 76.4448) (end 111.0856 75.8448) (width 0.127) (layer F.Cu) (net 20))
 (segment (start 110.4856 78.4448) (end 110.4856 76.4448) (width 0.127) (layer F.Cu) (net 20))
 (segment (start 111.0106 78.9698) (end 110.4856 78.4448) (width 0.127) (layer F.Cu) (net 20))
 (segment (start 112.0106 79.0448) (end 111.9356 78.9698) (width 0.127) (layer F.Cu) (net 20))
 (segment (start 109.6356 90.2448) (end 109.6356 87.7698) (width 0.127) (layer F.Cu) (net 22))
 (segment (start 109.6356 87.7698) (end 111.9356 85.4698) (width 0.127) (layer F.Cu) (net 22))
 (segment (start 111.4356 85.9698) (end 111.9356 85.4698) (width 0.127) (layer F.Cu) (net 22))
 (segment (start 113.9356 74.6448) (end 113.9356 74.9948) (width 0.127) (layer F.Cu) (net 21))
 (segment (start 113.9356 74.9948) (end 112.6856 76.2448) (width 0.127) (layer F.Cu) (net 21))
 (segment (start 112.6856 76.2448) (end 111.2856 76.2448) (width 0.127) (layer F.Cu) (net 21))
 (segment (start 111.2856 76.2448) (end 110.8856 76.6448) (width 0.127) (layer F.Cu) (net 21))
 (segment (start 110.8856 76.6448) (end 110.8856 78.0448) (width 0.127) (layer F.Cu) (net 21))
 (segment (start 110.8856 78.0448) (end 111.1606 78.3198) (width 0.127) (layer F.Cu) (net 21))
 (segment (start 111.1606 78.3198) (end 111.9356 78.3198) (width 0.127) (layer F.Cu) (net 21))
 (segment (start 112.0606 78.4448) (end 111.9356 78.3198) (width 0.127) (layer F.Cu) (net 21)))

